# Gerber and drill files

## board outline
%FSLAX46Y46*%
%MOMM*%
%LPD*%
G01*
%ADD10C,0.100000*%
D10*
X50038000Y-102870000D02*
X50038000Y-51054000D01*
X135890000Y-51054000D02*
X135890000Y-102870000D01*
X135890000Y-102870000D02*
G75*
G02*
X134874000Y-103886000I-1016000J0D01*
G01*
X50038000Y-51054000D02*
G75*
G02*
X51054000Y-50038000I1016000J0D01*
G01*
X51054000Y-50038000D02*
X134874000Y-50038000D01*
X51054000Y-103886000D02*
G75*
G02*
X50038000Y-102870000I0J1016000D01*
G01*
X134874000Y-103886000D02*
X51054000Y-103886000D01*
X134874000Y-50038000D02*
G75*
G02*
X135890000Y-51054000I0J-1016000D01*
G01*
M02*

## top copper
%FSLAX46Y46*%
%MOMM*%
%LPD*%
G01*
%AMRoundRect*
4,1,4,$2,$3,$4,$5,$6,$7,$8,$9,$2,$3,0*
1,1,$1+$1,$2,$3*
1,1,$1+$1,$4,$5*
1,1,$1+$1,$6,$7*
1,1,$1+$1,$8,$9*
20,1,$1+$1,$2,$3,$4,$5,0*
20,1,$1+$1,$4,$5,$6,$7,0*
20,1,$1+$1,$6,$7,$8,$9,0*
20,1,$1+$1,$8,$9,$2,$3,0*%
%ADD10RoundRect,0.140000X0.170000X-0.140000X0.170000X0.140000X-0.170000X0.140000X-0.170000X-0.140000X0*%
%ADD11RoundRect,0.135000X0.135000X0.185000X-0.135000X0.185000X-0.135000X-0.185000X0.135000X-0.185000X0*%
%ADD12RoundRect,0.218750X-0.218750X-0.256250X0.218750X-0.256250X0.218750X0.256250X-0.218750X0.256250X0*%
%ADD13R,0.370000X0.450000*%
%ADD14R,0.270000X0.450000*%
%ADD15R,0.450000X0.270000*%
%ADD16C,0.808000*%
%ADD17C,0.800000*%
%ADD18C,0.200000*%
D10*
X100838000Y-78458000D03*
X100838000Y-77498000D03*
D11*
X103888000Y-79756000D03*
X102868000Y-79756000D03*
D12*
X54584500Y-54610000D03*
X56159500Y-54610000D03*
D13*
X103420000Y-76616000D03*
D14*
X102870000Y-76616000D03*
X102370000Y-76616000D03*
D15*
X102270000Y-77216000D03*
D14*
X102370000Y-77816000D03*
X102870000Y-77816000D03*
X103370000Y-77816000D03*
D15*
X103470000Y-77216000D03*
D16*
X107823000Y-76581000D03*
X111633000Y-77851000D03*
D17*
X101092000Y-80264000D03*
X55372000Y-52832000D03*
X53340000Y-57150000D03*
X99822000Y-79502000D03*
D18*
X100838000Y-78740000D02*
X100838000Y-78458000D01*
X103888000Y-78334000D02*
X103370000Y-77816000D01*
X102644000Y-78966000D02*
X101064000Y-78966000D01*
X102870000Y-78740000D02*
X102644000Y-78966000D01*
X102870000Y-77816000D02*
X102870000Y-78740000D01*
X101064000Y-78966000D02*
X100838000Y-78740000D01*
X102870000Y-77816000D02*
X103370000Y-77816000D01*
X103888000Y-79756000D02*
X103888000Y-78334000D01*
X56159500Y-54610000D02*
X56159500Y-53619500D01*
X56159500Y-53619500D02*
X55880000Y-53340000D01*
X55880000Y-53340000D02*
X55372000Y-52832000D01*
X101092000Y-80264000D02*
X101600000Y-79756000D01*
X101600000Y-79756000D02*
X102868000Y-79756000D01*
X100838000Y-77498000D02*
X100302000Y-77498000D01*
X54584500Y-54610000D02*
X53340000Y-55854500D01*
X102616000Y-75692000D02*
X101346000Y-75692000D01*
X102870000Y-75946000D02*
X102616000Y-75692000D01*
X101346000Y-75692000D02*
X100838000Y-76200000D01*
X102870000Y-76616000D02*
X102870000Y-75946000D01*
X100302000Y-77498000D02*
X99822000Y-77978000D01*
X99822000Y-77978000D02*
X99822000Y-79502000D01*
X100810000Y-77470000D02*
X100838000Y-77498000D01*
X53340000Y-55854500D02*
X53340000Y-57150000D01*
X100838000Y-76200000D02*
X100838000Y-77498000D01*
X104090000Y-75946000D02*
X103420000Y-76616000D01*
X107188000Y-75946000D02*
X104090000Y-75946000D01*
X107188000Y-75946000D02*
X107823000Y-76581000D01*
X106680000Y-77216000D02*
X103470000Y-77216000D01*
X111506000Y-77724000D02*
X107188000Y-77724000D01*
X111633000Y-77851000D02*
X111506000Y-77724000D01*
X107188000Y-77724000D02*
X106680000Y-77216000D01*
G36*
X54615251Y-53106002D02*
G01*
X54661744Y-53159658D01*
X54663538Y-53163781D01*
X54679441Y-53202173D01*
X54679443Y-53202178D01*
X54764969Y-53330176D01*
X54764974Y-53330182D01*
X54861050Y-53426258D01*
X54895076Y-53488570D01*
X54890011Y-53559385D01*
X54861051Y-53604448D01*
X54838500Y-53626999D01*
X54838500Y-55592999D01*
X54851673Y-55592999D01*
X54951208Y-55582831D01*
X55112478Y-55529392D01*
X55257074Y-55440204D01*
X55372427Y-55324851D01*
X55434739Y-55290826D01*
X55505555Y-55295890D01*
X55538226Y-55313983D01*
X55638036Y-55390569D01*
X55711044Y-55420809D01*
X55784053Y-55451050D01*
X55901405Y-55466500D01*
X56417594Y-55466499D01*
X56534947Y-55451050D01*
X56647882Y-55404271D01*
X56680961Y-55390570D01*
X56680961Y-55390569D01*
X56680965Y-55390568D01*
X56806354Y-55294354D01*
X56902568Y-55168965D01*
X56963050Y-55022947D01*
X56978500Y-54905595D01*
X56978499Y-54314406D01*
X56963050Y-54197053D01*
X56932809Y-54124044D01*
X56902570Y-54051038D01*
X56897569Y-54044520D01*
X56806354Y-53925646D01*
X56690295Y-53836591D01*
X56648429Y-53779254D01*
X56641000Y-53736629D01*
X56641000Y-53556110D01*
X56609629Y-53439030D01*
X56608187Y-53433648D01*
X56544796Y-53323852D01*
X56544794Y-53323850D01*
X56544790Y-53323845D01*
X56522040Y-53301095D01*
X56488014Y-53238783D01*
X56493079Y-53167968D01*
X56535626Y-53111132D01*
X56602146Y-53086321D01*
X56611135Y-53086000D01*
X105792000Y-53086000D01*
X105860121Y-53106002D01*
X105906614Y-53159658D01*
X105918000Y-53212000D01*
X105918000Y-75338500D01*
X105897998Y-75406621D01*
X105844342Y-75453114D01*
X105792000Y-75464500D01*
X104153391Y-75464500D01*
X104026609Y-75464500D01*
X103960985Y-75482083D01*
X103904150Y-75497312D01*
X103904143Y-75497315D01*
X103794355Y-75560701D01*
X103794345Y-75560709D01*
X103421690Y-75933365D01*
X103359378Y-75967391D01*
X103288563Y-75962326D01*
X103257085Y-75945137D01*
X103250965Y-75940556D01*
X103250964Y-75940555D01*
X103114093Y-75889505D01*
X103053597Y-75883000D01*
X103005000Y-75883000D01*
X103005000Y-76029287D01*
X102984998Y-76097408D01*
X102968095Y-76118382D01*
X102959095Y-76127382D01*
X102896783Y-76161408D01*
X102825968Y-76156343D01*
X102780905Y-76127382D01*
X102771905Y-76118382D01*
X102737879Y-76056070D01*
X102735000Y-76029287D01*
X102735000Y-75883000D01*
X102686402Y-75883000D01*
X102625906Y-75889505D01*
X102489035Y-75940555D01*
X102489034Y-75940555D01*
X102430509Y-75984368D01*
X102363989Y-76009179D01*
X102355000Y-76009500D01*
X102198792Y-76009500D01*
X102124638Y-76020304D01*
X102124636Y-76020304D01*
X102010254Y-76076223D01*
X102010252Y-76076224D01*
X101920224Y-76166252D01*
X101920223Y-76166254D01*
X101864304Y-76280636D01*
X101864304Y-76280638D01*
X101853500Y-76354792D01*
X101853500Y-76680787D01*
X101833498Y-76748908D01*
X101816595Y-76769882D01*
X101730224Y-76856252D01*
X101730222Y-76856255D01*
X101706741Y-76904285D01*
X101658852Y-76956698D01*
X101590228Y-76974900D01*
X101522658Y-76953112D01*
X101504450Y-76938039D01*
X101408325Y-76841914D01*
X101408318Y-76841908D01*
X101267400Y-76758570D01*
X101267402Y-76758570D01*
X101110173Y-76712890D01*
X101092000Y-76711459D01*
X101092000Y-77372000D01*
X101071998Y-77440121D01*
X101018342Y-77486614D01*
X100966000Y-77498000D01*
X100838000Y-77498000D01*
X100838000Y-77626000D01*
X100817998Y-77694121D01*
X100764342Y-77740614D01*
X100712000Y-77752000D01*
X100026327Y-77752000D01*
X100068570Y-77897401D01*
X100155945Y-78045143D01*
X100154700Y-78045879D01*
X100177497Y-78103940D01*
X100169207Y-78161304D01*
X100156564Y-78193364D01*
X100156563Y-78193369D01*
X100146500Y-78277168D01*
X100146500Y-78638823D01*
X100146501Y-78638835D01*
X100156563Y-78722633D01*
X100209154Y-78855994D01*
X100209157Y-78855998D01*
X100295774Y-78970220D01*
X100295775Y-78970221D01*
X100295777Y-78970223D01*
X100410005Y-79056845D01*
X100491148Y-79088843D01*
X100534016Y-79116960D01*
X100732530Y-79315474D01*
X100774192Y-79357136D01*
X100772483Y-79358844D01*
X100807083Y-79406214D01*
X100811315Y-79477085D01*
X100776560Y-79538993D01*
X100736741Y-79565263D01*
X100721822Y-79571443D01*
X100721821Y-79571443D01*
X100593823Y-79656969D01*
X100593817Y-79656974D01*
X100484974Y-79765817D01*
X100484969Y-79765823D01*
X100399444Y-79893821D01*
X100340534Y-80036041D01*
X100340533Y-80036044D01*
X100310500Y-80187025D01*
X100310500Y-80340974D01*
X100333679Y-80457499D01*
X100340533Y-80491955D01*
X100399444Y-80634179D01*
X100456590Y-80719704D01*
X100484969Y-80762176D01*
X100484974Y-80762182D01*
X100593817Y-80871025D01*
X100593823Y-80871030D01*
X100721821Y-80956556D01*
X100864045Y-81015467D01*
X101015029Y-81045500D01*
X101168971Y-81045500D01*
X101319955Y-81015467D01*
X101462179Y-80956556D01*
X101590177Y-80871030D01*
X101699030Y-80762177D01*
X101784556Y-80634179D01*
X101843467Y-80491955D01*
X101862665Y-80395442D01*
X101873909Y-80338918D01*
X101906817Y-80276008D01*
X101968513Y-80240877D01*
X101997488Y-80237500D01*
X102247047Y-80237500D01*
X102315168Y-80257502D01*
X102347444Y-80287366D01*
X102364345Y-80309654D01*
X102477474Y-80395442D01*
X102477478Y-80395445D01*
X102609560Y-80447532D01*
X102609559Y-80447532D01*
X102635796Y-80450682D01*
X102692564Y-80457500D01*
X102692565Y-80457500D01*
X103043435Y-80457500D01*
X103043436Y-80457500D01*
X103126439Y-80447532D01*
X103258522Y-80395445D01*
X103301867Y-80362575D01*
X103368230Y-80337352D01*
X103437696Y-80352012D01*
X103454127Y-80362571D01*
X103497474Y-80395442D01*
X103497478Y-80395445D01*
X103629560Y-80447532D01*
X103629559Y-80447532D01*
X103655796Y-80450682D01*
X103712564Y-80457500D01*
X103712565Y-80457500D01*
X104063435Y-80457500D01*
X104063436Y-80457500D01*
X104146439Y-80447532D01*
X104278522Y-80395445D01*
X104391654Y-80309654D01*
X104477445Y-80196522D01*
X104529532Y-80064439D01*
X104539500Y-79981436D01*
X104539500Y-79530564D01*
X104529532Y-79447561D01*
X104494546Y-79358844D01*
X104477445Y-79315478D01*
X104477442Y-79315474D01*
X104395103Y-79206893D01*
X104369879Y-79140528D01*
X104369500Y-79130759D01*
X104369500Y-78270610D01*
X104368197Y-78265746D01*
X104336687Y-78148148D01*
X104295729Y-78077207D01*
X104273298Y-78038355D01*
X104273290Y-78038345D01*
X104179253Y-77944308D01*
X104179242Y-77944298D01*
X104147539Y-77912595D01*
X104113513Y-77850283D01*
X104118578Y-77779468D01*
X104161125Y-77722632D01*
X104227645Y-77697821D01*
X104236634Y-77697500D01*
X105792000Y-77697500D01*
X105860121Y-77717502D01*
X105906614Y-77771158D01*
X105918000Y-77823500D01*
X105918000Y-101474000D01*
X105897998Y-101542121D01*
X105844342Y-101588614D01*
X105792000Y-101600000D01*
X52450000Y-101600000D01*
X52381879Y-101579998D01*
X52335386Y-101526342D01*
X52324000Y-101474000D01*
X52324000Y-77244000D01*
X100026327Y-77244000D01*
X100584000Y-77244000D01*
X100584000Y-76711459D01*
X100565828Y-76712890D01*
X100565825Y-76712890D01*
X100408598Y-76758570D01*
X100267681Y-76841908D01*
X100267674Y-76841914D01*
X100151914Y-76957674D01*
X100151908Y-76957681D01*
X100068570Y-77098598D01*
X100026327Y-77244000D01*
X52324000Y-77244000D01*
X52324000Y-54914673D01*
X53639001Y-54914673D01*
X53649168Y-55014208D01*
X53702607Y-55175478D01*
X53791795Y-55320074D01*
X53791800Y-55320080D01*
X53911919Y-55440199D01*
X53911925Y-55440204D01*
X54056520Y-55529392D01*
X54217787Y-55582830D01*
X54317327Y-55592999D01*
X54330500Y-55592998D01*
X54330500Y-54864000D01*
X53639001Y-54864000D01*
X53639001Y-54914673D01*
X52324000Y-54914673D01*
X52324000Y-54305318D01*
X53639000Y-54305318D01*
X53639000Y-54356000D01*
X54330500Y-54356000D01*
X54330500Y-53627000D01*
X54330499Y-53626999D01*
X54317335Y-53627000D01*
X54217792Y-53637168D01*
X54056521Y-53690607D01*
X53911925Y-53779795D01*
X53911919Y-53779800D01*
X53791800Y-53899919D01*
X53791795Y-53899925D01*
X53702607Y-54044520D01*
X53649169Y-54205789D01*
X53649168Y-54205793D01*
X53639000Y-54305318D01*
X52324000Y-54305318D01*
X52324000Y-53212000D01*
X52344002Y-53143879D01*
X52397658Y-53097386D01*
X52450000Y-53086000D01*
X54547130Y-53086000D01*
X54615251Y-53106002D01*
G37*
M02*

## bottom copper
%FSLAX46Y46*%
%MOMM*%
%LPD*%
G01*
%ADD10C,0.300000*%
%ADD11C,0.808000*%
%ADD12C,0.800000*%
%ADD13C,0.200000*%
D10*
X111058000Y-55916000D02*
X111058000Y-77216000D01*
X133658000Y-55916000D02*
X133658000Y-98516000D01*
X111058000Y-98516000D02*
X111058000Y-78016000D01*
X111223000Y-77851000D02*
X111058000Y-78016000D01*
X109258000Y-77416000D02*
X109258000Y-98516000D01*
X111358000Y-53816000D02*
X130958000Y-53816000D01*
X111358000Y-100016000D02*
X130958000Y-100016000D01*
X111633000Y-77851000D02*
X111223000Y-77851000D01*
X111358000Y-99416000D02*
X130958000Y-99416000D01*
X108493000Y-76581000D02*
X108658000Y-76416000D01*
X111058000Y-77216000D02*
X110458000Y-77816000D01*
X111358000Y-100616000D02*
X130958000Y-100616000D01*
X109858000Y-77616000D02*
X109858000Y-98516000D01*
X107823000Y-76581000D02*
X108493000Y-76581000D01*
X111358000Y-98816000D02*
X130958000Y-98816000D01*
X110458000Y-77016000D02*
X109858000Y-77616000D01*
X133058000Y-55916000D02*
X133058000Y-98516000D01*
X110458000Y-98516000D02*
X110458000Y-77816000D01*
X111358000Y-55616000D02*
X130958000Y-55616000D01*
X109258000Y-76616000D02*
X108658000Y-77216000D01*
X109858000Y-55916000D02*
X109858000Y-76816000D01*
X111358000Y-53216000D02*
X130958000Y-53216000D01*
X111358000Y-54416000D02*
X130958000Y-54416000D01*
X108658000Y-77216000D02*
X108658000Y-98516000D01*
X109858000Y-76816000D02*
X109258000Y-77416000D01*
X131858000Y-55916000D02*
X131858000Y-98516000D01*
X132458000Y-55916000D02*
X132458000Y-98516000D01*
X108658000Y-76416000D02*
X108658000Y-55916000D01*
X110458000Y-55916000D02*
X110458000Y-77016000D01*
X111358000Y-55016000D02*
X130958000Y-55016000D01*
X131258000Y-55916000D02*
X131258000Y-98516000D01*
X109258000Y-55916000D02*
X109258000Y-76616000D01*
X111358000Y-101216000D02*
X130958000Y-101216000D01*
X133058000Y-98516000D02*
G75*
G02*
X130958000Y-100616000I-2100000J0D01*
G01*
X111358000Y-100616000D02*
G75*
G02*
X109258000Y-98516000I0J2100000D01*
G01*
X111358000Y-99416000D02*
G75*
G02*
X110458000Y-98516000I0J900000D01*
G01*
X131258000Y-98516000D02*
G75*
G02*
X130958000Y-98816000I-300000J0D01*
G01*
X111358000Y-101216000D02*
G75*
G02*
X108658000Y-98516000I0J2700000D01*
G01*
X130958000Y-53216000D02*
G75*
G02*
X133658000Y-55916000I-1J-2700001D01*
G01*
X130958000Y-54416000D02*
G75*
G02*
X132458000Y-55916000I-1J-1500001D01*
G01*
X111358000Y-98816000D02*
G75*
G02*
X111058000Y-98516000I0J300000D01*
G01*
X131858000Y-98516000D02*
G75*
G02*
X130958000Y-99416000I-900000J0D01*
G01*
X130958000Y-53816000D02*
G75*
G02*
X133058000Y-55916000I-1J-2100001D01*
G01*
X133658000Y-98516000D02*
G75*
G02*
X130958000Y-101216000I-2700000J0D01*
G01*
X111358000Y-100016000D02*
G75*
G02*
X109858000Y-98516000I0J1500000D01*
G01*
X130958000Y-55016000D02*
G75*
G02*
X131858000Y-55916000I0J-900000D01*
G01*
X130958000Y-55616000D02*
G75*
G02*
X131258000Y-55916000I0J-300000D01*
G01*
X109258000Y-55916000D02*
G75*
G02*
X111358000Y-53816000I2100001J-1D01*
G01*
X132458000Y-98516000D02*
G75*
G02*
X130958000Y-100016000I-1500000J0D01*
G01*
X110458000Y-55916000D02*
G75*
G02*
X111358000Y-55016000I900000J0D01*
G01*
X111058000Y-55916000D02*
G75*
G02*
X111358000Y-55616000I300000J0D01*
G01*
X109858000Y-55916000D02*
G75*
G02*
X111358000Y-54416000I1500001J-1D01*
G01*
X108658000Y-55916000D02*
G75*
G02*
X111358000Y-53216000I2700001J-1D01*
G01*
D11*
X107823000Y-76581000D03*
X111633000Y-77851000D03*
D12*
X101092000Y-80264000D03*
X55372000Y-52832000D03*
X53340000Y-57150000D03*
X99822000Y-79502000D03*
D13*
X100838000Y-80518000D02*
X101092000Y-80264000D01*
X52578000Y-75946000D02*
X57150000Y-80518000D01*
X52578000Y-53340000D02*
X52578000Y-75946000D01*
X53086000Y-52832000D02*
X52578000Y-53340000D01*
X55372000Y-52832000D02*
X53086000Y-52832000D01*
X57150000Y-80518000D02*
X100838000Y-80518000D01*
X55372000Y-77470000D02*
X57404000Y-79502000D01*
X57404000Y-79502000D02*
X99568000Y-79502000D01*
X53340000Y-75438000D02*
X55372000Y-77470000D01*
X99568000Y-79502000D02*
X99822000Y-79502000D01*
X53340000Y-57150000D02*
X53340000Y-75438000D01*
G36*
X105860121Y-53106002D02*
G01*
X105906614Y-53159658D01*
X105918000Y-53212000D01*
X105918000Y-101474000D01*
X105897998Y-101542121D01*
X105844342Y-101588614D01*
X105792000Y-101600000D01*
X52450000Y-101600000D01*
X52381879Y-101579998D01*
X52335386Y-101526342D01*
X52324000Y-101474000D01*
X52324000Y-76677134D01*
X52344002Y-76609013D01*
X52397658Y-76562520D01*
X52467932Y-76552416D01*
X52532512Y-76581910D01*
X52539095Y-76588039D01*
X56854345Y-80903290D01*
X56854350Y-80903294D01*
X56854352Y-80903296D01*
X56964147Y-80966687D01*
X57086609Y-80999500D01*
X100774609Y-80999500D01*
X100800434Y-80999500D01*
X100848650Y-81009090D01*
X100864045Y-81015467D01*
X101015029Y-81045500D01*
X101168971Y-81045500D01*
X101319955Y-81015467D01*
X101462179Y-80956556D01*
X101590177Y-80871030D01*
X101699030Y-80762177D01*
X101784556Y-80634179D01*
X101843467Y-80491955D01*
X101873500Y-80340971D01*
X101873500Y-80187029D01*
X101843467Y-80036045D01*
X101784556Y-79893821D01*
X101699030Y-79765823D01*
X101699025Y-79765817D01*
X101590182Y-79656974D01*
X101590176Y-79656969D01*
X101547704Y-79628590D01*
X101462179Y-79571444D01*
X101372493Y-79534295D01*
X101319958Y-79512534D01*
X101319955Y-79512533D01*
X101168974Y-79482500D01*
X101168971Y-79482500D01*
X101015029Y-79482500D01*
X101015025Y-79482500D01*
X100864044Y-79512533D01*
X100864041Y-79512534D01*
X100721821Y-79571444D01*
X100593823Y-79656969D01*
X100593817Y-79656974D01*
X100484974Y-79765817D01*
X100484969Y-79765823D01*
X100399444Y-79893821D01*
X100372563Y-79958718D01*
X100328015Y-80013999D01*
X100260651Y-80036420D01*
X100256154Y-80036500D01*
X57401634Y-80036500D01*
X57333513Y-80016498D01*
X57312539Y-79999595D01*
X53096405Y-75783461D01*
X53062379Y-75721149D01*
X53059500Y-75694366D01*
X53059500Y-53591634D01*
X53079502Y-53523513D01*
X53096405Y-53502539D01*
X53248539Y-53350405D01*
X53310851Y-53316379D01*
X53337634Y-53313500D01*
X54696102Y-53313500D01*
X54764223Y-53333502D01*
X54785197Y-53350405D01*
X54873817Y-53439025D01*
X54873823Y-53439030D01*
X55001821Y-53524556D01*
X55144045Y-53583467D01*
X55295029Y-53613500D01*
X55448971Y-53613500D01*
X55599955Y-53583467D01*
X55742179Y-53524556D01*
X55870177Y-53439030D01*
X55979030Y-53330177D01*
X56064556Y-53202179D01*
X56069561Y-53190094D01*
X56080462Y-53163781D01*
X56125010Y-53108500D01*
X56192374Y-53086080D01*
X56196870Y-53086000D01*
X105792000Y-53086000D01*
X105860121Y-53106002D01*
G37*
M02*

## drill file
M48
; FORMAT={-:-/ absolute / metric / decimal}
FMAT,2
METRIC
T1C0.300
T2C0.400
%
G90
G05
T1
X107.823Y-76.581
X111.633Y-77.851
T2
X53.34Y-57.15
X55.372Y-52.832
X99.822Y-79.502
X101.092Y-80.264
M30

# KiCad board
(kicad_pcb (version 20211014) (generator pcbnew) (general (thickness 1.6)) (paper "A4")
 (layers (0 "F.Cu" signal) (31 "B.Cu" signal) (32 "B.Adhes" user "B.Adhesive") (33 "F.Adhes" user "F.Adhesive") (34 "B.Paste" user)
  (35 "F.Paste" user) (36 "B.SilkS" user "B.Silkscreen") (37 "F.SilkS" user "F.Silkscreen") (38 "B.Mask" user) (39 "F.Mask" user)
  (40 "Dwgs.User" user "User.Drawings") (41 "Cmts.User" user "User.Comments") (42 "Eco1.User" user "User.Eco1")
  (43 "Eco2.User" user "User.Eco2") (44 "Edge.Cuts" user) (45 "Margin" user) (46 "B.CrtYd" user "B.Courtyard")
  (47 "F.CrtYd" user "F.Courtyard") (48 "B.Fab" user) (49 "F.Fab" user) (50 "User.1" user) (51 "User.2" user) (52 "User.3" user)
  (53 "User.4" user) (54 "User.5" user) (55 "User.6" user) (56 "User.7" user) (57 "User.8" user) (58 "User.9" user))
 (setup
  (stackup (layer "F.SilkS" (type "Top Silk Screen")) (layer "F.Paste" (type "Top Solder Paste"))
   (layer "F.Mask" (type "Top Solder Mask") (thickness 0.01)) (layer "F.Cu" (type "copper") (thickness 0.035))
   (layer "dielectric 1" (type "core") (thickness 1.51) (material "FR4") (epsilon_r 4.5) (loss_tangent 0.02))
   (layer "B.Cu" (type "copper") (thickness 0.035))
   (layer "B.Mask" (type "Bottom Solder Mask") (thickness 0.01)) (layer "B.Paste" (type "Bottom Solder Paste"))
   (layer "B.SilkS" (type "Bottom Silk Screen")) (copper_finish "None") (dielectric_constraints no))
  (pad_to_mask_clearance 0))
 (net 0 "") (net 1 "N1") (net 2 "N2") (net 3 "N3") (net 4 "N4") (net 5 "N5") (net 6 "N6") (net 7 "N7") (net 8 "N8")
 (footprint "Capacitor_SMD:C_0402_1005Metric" (layer "F.Cu") (at 100.838 77.978 90)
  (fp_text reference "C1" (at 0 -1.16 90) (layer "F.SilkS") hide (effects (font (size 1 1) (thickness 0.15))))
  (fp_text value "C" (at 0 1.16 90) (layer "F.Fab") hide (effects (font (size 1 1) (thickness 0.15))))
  (pad "1" smd roundrect locked (at -0.48 0 90) (size 0.56 0.62) (layers "F.Cu" "F.Paste" "F.Mask") (roundrect_rratio 0.25) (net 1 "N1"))
  (pad "2" smd roundrect locked (at 0.48 0 90) (size 0.56 0.62) (layers "F.Cu" "F.Paste" "F.Mask") (roundrect_rratio 0.25) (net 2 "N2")))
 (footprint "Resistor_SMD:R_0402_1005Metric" (layer "F.Cu") (at 103.378 79.756 180)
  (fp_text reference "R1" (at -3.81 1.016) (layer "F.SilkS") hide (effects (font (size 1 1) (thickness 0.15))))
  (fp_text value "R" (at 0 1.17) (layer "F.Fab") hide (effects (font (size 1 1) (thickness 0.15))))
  (pad "1" smd roundrect locked (at -0.51 0 180) (size 0.54 0.64) (layers "F.Cu" "F.Paste" "F.Mask") (roundrect_rratio 0.25) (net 1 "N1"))
  (pad "2" smd roundrect locked (at 0.51 0 180) (size 0.54 0.64) (layers "F.Cu" "F.Paste" "F.Mask") (roundrect_rratio 0.25) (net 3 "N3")))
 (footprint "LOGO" (layer "F.Cu") (at 109.733787 79.156487)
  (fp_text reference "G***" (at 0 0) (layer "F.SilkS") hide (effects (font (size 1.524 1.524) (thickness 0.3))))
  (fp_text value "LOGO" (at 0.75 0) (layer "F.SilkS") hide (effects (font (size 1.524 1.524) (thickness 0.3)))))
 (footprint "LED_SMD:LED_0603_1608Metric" (layer "F.Cu") (at 55.372 54.61)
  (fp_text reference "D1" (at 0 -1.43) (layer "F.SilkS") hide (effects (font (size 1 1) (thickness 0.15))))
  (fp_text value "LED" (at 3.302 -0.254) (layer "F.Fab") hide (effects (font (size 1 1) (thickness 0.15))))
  (pad "1" smd roundrect locked (at -0.7875 0) (size 0.875 0.95) (layers "F.Cu" "F.Paste" "F.Mask") (roundrect_rratio 0.25) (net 2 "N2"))
  (pad "2" smd roundrect locked (at 0.7875 0) (size 0.875 0.95) (layers "F.Cu" "F.Paste" "F.Mask") (roundrect_rratio 0.25) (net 3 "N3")))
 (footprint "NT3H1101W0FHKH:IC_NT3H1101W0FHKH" (layer "F.Cu") (at 102.87 77.216 -90)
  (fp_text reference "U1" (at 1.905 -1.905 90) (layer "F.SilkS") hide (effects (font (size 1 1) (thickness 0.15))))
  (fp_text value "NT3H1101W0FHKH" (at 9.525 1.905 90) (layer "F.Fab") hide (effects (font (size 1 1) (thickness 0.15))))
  (pad "1" smd rect locked (at -0.6 -0.55 90) (size 0.45 0.37) (layers "F.Cu" "F.Mask") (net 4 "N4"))
  (pad "2" smd rect locked (at -0.6 0 90) (size 0.45 0.27) (layers "F.Cu" "F.Mask") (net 2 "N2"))
  (pad "3" smd rect locked (at -0.6 0.5 90) (size 0.45 0.27) (layers "F.Cu" "F.Mask") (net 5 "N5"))
  (pad "4" smd rect locked (at 0 0.6 180) (size 0.45 0.27) (layers "F.Cu" "F.Mask") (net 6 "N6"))
  (pad "5" smd rect locked (at 0.6 0.5 90) (size 0.45 0.27) (layers "F.Cu" "F.Mask") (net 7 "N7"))
  (pad "6" smd rect locked (at 0.6 0 90) (size 0.45 0.27) (layers "F.Cu" "F.Mask") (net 1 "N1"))
  (pad "7" smd rect locked (at 0.6 -0.5 90) (size 0.45 0.27) (layers "F.Cu" "F.Mask") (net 1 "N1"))
  (pad "8" smd rect locked (at 0 -0.6 180) (size 0.45 0.27) (layers "F.Cu" "F.Mask") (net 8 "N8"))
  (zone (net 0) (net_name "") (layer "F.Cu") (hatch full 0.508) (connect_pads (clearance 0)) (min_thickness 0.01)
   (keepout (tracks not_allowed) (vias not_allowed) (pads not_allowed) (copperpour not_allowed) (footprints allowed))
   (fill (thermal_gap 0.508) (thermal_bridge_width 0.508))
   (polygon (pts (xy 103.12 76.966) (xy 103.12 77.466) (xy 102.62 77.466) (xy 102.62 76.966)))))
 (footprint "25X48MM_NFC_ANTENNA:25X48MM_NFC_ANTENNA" (layer "B.Cu") (at 121.158 77.216 -90)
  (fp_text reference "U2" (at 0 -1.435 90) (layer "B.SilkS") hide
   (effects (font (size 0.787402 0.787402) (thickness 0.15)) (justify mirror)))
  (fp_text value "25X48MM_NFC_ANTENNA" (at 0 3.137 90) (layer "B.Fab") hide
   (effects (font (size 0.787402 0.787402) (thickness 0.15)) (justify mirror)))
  (fp_line (start -21.3 10.1) (end 0 10.1) (layer "B.Cu") (width 0.3))
  (fp_line (start -21.3 -12.5) (end 21.3 -12.5) (layer "B.Cu") (width 0.3))
  (fp_line (start 21.3 10.1) (end 0.8 10.1) (layer "B.Cu") (width 0.3))
  (fp_line (start 0.635 9.935) (end 0.8 10.1) (layer "B.Cu") (width 0.3))
  (fp_line (start 0.2 11.9) (end 21.3 11.9) (layer "B.Cu") (width 0.3))
  (fp_line (start -23.4 9.8) (end -23.4 -9.8) (layer "B.Cu") (width 0.3))
  (fp_line (start 22.8 9.8) (end 22.8 -9.8) (layer "B.Cu") (width 0.3))
  (fp_line (start 0.635 9.525) (end 0.635 9.935) (layer "B.Cu") (width 0.3))
  (fp_line (start 22.2 9.8) (end 22.2 -9.8) (layer "B.Cu") (width 0.3))
  (fp_line (start -0.635 12.665) (end -0.8 12.5) (layer "B.Cu") (width 0.3))
  (fp_line (start 0 10.1) (end 0.6 10.7) (layer "B.Cu") (width 0.3))
  (fp_line (start 23.4 9.8) (end 23.4 -9.8) (layer "B.Cu") (width 0.3))
  (fp_line (start 0.4 11.3) (end 21.3 11.3) (layer "B.Cu") (width 0.3))
  (fp_line (start -0.635 13.335) (end -0.635 12.665) (layer "B.Cu") (width 0.3))
  (fp_line (start 21.6 9.8) (end 21.6 -9.8) (layer "B.Cu") (width 0.3))
  (fp_line (start -0.2 10.7) (end 0.4 11.3) (layer "B.Cu") (width 0.3))
  (fp_line (start -21.3 -11.9) (end 21.3 -11.9) (layer "B.Cu") (width 0.3))
  (fp_line (start 21.3 10.7) (end 0.6 10.7) (layer "B.Cu") (width 0.3))
  (fp_line (start -21.6 9.8) (end -21.6 -9.8) (layer "B.Cu") (width 0.3))
  (fp_line (start -0.6 11.9) (end 0 12.5) (layer "B.Cu") (width 0.3))
  (fp_line (start -21.3 11.3) (end -0.4 11.3) (layer "B.Cu") (width 0.3))
  (fp_line (start -24 9.8) (end -24 -9.8) (layer "B.Cu") (width 0.3))
  (fp_line (start -22.8 9.8) (end -22.8 -9.8) (layer "B.Cu") (width 0.3))
  (fp_line (start 0 12.5) (end 21.3 12.5) (layer "B.Cu") (width 0.3))
  (fp_line (start -0.4 11.3) (end 0.2 11.9) (layer "B.Cu") (width 0.3))
  (fp_line (start -21.3 -10.7) (end 21.3 -10.7) (layer "B.Cu") (width 0.3))
  (fp_line (start -21.3 -11.3) (end 21.3 -11.3) (layer "B.Cu") (width 0.3))
  (fp_line (start -0.8 12.5) (end -21.3 12.5) (layer "B.Cu") (width 0.3))
  (fp_line (start -21.3 10.7) (end -0.2 10.7) (layer "B.Cu") (width 0.3))
  (fp_line (start -22.2 9.8) (end -22.2 -9.8) (layer "B.Cu") (width 0.3))
  (fp_line (start -21.3 -10.1) (end 21.3 -10.1) (layer "B.Cu") (width 0.3))
  (fp_line (start -21.3 11.9) (end -0.6 11.9) (layer "B.Cu") (width 0.3))
  (fp_line (start 24 9.8) (end 24 -9.8) (layer "B.Cu") (width 0.3))
  (fp_arc (start 21.3 -11.9) (mid 22.784924 -11.284924) (end 23.4 -9.8) (layer "B.Cu") (width 0.3))
  (fp_arc (start 23.4 9.8) (mid 22.784924 11.284924) (end 21.3 11.9) (layer "B.Cu") (width 0.3))
  (fp_arc (start 22.2 9.8) (mid 21.936396 10.436396) (end 21.3 10.7) (layer "B.Cu") (width 0.3))
  (fp_arc (start 21.3 -10.1) (mid 21.512132 -10.012132) (end 21.6 -9.8) (layer "B.Cu") (width 0.3))
  (fp_arc (start 24 9.8) (mid 23.209188 11.709188) (end 21.3 12.5) (layer "B.Cu") (width 0.3))
  (fp_arc (start -24 -9.8) (mid -23.209188 -11.709188) (end -21.3 -12.5) (layer "B.Cu") (width 0.3))
  (fp_arc (start -22.8 -9.8) (mid -22.36066 -10.86066) (end -21.3 -11.3) (layer "B.Cu") (width 0.3))
  (fp_arc (start 21.6 9.8) (mid 21.512132 10.012132) (end 21.3 10.1) (layer "B.Cu") (width 0.3))
  (fp_arc (start 21.3 -10.7) (mid 21.936396 -10.436396) (end 22.2 -9.8) (layer "B.Cu") (width 0.3))
  (fp_arc (start -23.4 -9.8) (mid -22.784924 -11.284924) (end -21.3 -11.9) (layer "B.Cu") (width 0.3))
  (fp_arc (start 21.3 -12.5) (mid 23.209188 -11.709188) (end 24 -9.8) (layer "B.Cu") (width 0.3))
  (fp_arc (start 22.8 9.8) (mid 22.36066 10.86066) (end 21.3 11.3) (layer "B.Cu") (width 0.3))
  (fp_arc (start -22.2 -9.8) (mid -21.936396 -10.436396) (end -21.3 -10.7) (layer "B.Cu") (width 0.3))
  (fp_arc (start -21.6 -9.8) (mid -21.512132 -10.012132) (end -21.3 -10.1) (layer "B.Cu") (width 0.3))
  (fp_arc (start -21.3 11.9) (mid -22.784924 11.284924) (end -23.4 9.8) (layer "B.Cu") (width 0.3))
  (fp_arc (start 21.3 -11.3) (mid 22.36066 -10.86066) (end 22.8 -9.8) (layer "B.Cu") (width 0.3))
  (fp_arc (start -21.3 10.7) (mid -21.936396 10.436396) (end -22.2 9.8) (layer "B.Cu") (width 0.3))
  (fp_arc (start -21.3 10.1) (mid -21.512132 10.012132) (end -21.6 9.8) (layer "B.Cu") (width 0.3))
  (fp_arc (start -21.3 11.3) (mid -22.36066 10.86066) (end -22.8 9.8) (layer "B.Cu") (width 0.3))
  (fp_arc (start -21.3 12.5) (mid -23.209188 11.709188) (end -24 9.8) (layer "B.Cu") (width 0.3))
  (pad "P$1" thru_hole circle (at -0.635 13.335 270) (size 0.808 0.808) (drill 0.3) (layers *.Cu *.Mask) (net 4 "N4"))
  (pad "P$2" thru_hole circle (at 0.635 9.525 270) (size 0.808 0.808) (drill 0.3) (layers *.Cu *.Mask) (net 8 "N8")))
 (gr_line (start 50.038 102.87) (end 50.038 51.054) (layer "Edge.Cuts") (width 0.1))
 (gr_line (start 135.89 51.054) (end 135.89 102.87) (layer "Edge.Cuts") (width 0.1))
 (gr_arc (start 135.89 102.87) (mid 135.59242 103.58842) (end 134.874 103.886) (layer "Edge.Cuts") (width 0.1))
 (gr_arc (start 50.038 51.054) (mid 50.33558 50.33558) (end 51.054 50.038) (layer "Edge.Cuts") (width 0.1))
 (gr_line (start 51.054 50.038) (end 134.874 50.038) (layer "Edge.Cuts") (width 0.1))
 (gr_arc (start 51.054 103.886) (mid 50.33558 103.58842) (end 50.038 102.87) (layer "Edge.Cuts") (width 0.1))
 (gr_line (start 134.874 103.886) (end 51.054 103.886) (layer "Edge.Cuts") (width 0.1))
 (gr_arc (start 134.874 50.038) (mid 135.59242 50.33558) (end 135.89 51.054) (layer "Edge.Cuts") (width 0.1))
 (segment (start 100.838 78.74) (end 100.838 78.458) (width 0.2) (layer "F.Cu") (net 1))
 (segment (start 103.888 78.334) (end 103.37 77.816) (width 0.2) (layer "F.Cu") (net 1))
 (segment (start 102.644 78.966) (end 101.064 78.966) (width 0.2) (layer "F.Cu") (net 1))
 (segment (start 102.87 78.74) (end 102.644 78.966) (width 0.2) (layer "F.Cu") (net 1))
 (segment (start 102.87 77.816) (end 102.87 78.74) (width 0.2) (layer "F.Cu") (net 1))
 (segment (start 101.064 78.966) (end 100.838 78.74) (width 0.2) (layer "F.Cu") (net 1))
 (segment (start 102.87 77.816) (end 103.37 77.816) (width 0.2) (layer "F.Cu") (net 1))
 (segment (start 103.888 79.756) (end 103.888 78.334) (width 0.2) (layer "F.Cu") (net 1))
 (segment (start 56.1595 54.61) (end 56.1595 53.6195) (width 0.2) (layer "F.Cu") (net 3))
 (segment (start 56.1595 53.6195) (end 55.88 53.34) (width 0.2) (layer "F.Cu") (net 3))
 (segment (start 55.88 53.34) (end 55.372 52.832) (width 0.2) (layer "F.Cu") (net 3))
 (segment (start 101.092 80.264) (end 101.6 79.756) (width 0.2) (layer "F.Cu") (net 3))
 (segment (start 101.6 79.756) (end 102.868 79.756) (width 0.2) (layer "F.Cu") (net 3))
 (via (at 101.092 80.264) (size 0.8) (drill 0.4) (layers "F.Cu" "B.Cu") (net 3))
 (via (at 55.372 52.832) (size 0.8) (drill 0.4) (layers "F.Cu" "B.Cu") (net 3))
 (segment (start 100.838 80.518) (end 101.092 80.264) (width 0.2) (layer "B.Cu") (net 3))
 (segment (start 52.578 75.946) (end 57.15 80.518) (width 0.2) (layer "B.Cu") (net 3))
 (segment (start 52.578 53.34) (end 52.578 75.946) (width 0.2) (layer "B.Cu") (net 3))
 (segment (start 53.086 52.832) (end 52.578 53.34) (width 0.2) (layer "B.Cu") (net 3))
 (segment (start 55.372 52.832) (end 53.086 52.832) (width 0.2) (layer "B.Cu") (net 3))
 (segment (start 57.15 80.518) (end 100.838 80.518) (width 0.2) (layer "B.Cu") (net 3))
 (segment (start 100.838 77.498) (end 100.302 77.498) (width 0.2) (layer "F.Cu") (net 2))
 (segment (start 54.5845 54.61) (end 53.34 55.8545) (width 0.2) (layer "F.Cu") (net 2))
 (segment (start 102.616 75.692) (end 101.346 75.692) (width 0.2) (layer "F.Cu") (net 2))
 (segment (start 102.87 75.946) (end 102.616 75.692) (width 0.2) (layer "F.Cu") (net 2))
 (segment (start 101.346 75.692) (end 100.838 76.2) (width 0.2) (layer "F.Cu") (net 2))
 (segment (start 102.87 76.616) (end 102.87 75.946) (width 0.2) (layer "F.Cu") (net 2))
 (segment (start 100.302 77.498) (end 99.822 77.978) (width 0.2) (layer "F.Cu") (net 2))
 (segment (start 99.822 77.978) (end 99.822 79.502) (width 0.2) (layer "F.Cu") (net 2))
 (segment (start 100.81 77.47) (end 100.838 77.498) (width 0.2) (layer "F.Cu") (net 2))
 (segment (start 53.34 55.8545) (end 53.34 57.15) (width 0.2) (layer "F.Cu") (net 2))
 (segment (start 100.838 76.2) (end 100.838 77.498) (width 0.2) (layer "F.Cu") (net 2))
 (via (at 53.34 57.15) (size 0.8) (drill 0.4) (layers "F.Cu" "B.Cu") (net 2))
 (via (at 99.822 79.502) (size 0.8) (drill 0.4) (layers "F.Cu" "B.Cu") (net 2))
 (segment (start 55.372 77.47) (end 57.404 79.502) (width 0.2) (layer "B.Cu") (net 2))
 (segment (start 57.404 79.502) (end 99.568 79.502) (width 0.2) (layer "B.Cu") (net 2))
 (segment (start 53.34 75.438) (end 55.372 77.47) (width 0.2) (layer "B.Cu") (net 2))
 (segment (start 99.568 79.502) (end 99.822 79.502) (width 0.2) (layer "B.Cu") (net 2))
 (segment (start 53.34 57.15) (end 53.34 75.438) (width 0.2) (layer "B.Cu") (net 2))
 (segment (start 104.09 75.946) (end 103.42 76.616) (width 0.2) (layer "F.Cu") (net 4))
 (segment (start 107.188 75.946) (end 104.09 75.946) (width 0.2) (layer "F.Cu") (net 4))
 (segment (start 107.188 75.946) (end 107.823 76.581) (width 0.2) (layer "F.Cu") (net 4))
 (segment (start 106.68 77.216) (end 103.47 77.216) (width 0.2) (layer "F.Cu") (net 8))
 (segment (start 111.506 77.724) (end 107.188 77.724) (width 0.2) (layer "F.Cu") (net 8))
 (segment (start 111.633 77.851) (end 111.506 77.724) (width 0.2) (layer "F.Cu") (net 8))
 (segment (start 107.188 77.724) (end 106.68 77.216) (width 0.2) (layer "F.Cu") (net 8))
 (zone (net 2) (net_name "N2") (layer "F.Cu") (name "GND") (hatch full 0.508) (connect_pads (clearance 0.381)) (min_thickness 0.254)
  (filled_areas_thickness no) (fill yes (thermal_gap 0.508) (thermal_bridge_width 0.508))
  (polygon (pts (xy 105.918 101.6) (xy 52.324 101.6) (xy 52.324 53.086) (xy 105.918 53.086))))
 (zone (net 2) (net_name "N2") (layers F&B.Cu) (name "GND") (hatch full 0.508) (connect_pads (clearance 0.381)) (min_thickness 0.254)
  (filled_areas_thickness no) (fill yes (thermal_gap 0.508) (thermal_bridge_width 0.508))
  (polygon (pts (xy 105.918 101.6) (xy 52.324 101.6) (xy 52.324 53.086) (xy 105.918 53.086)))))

